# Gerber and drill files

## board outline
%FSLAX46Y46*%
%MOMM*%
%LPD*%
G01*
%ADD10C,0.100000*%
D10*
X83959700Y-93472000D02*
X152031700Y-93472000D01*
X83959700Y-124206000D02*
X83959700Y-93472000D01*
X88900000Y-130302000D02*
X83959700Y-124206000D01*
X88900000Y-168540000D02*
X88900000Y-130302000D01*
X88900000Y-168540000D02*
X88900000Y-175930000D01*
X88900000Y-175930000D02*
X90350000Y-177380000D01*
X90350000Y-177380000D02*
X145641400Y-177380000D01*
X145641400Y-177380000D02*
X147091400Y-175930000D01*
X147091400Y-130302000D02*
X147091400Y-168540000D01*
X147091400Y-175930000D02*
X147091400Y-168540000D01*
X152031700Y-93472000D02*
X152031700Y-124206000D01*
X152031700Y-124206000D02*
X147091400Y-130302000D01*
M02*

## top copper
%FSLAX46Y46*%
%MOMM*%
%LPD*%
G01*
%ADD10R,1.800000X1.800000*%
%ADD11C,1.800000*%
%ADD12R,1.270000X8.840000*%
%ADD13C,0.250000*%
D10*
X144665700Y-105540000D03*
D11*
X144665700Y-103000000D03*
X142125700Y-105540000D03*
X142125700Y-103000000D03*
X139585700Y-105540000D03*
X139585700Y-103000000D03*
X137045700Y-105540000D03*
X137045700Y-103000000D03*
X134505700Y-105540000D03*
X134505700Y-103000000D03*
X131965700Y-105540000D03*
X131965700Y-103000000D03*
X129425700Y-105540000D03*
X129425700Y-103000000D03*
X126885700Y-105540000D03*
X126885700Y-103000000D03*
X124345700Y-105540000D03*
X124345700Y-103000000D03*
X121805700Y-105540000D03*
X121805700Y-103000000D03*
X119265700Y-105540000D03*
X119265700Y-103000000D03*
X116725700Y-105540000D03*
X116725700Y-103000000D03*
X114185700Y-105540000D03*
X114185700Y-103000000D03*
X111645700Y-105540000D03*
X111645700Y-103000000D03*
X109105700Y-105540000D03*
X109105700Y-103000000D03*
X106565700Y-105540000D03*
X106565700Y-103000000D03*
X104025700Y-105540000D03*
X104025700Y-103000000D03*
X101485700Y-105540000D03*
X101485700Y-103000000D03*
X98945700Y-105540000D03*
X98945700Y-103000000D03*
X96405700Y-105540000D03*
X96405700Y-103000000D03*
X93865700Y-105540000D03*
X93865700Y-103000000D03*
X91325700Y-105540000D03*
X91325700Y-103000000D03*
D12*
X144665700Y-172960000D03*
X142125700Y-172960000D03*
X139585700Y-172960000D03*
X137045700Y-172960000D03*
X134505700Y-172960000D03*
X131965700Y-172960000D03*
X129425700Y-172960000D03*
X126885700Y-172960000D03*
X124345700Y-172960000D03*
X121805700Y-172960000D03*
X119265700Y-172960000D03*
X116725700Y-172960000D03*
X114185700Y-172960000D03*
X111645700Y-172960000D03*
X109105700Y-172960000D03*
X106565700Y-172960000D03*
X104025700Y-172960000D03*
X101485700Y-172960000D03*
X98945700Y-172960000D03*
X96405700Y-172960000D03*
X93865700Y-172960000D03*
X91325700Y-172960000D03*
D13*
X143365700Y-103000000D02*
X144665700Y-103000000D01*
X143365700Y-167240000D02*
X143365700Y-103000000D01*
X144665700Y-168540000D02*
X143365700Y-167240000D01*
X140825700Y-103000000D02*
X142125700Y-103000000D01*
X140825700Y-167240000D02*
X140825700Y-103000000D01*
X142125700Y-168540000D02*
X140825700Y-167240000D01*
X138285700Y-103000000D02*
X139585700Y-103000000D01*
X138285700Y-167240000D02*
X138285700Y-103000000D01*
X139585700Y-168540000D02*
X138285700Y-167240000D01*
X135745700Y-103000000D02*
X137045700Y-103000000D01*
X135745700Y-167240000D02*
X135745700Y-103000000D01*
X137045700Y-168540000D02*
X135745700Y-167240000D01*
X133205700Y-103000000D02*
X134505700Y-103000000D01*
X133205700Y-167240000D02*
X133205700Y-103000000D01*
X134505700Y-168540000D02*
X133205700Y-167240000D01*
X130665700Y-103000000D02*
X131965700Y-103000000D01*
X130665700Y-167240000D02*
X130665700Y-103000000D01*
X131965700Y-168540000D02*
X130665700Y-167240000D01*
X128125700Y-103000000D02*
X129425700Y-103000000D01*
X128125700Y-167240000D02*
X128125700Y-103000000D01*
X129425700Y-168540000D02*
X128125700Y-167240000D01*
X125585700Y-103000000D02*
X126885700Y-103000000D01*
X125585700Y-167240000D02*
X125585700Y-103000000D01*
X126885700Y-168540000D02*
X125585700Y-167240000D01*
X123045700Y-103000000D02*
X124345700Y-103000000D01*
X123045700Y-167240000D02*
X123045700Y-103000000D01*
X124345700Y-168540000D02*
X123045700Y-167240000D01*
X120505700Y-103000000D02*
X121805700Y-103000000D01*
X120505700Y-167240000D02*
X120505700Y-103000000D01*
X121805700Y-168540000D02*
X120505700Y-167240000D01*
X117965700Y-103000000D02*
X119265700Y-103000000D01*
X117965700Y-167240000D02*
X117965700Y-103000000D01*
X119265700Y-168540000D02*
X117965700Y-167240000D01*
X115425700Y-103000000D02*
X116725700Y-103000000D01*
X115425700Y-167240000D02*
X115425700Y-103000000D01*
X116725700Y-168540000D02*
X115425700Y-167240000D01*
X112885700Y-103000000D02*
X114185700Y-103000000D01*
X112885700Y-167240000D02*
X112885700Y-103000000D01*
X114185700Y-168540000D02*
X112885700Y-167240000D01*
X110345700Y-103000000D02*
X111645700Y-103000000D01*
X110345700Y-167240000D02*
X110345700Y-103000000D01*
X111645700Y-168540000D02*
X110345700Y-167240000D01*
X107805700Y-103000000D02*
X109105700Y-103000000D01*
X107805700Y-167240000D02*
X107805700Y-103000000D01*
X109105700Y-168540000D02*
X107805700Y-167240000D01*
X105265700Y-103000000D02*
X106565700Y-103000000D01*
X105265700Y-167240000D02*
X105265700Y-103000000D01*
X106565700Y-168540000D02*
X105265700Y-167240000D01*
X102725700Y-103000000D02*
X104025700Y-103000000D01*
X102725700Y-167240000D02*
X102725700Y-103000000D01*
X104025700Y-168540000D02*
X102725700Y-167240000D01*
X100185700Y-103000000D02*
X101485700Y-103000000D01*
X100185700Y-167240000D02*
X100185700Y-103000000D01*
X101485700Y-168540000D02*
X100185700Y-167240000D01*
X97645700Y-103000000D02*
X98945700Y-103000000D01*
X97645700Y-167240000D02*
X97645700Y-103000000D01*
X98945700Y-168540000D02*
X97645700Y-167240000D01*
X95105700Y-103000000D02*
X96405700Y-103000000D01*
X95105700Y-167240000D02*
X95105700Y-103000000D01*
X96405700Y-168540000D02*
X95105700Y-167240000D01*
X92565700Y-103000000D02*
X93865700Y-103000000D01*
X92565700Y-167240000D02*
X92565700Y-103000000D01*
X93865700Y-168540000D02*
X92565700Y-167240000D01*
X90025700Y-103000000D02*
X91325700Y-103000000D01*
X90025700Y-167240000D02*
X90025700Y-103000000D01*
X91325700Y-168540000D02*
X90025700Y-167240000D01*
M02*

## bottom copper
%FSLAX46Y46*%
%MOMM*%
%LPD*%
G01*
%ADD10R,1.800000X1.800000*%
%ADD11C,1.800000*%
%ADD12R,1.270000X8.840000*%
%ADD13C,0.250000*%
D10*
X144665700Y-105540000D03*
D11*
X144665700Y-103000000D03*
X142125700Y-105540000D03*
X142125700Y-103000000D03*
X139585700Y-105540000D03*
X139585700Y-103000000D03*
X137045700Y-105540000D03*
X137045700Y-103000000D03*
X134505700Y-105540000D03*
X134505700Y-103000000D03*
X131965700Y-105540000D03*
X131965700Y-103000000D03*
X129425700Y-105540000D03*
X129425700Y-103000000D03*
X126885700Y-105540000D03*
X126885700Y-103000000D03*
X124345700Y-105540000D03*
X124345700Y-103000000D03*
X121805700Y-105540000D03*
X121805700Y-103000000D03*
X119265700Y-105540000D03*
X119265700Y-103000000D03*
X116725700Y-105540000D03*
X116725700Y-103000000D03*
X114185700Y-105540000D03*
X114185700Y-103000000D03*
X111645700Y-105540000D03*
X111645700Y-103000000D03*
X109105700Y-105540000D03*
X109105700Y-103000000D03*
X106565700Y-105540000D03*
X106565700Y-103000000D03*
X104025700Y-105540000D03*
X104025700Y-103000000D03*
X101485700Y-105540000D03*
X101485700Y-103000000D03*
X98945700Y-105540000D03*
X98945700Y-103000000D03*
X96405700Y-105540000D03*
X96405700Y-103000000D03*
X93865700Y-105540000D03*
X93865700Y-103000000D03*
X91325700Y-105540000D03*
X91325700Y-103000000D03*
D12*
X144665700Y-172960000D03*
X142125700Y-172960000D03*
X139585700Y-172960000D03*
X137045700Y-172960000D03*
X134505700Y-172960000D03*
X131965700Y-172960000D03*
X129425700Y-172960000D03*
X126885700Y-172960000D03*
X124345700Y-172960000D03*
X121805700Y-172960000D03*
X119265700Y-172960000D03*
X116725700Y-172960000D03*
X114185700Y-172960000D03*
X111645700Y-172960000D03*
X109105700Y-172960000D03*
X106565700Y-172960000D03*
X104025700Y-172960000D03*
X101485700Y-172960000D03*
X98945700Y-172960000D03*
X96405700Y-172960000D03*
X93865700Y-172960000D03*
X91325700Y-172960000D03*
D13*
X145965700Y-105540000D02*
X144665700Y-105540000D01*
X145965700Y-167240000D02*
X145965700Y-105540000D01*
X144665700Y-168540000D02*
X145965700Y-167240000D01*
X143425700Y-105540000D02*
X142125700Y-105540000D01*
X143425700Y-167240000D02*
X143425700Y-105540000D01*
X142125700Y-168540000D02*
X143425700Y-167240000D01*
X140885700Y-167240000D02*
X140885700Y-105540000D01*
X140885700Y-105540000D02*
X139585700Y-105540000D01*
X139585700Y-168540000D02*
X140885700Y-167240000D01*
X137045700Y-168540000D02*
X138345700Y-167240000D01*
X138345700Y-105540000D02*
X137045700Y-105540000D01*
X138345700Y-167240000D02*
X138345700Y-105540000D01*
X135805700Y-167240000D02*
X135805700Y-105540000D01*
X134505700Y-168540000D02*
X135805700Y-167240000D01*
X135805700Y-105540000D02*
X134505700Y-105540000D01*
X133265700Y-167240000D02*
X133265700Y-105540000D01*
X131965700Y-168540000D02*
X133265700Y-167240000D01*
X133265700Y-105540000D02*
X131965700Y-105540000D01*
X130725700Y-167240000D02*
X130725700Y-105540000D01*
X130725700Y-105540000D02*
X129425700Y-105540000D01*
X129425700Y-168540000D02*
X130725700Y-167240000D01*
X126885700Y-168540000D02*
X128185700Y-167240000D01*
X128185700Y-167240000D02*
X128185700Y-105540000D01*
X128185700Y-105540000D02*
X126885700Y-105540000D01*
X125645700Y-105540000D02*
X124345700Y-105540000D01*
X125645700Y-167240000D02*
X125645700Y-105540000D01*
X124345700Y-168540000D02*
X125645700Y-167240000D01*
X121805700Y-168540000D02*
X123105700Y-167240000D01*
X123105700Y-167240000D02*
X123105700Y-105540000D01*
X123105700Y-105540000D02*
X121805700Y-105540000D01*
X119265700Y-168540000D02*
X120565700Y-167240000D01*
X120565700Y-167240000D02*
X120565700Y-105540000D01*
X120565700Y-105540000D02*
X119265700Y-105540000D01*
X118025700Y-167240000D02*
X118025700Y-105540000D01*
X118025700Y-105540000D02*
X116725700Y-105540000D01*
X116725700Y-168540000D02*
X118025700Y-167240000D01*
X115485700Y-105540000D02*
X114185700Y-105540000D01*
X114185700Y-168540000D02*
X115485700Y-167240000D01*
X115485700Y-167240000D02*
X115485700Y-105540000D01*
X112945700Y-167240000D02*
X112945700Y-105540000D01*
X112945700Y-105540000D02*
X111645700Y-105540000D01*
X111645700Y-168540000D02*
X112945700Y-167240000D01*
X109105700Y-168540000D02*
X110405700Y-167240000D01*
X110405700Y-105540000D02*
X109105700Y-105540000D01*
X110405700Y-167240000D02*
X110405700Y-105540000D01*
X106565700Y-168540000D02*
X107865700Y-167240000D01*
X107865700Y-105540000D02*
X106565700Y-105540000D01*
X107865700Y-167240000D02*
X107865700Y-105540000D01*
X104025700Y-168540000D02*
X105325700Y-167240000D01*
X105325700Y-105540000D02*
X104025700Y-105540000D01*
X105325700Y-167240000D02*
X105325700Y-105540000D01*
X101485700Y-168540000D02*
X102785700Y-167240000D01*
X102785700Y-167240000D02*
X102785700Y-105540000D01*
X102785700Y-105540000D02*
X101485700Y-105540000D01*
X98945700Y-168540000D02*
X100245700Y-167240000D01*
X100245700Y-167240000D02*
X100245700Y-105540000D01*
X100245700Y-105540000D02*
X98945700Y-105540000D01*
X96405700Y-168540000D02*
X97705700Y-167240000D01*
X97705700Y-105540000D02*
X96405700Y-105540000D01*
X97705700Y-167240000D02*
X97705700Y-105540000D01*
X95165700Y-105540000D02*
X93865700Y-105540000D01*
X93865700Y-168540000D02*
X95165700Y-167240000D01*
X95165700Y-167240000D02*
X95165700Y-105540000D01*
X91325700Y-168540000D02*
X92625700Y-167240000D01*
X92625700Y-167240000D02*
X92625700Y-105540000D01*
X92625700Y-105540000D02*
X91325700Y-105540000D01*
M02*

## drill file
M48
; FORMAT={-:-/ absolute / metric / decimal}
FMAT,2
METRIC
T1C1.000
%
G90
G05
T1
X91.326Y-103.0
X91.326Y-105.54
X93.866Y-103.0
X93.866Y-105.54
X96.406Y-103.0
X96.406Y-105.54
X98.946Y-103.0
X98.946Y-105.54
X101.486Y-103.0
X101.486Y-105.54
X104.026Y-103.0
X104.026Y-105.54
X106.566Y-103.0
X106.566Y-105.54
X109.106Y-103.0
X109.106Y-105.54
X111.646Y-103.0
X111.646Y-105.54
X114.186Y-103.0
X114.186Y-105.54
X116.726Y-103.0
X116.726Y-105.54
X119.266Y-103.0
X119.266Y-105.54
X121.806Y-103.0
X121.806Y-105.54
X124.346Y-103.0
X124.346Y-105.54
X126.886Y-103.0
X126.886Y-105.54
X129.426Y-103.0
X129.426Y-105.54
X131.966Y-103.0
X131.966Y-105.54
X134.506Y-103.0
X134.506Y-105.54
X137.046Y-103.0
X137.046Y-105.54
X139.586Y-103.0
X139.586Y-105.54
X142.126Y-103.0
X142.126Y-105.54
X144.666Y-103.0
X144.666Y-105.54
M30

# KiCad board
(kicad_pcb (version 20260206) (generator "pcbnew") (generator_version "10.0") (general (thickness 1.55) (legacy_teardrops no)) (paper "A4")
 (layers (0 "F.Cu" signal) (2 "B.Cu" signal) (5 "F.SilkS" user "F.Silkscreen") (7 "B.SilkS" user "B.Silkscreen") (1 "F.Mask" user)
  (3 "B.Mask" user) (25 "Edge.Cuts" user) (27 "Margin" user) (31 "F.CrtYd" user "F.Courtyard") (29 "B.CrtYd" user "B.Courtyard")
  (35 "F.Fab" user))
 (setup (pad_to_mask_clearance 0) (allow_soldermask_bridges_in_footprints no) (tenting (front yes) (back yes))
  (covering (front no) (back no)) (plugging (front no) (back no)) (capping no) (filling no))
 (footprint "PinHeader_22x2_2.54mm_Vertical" (layer "F.Cu") (at 0 0)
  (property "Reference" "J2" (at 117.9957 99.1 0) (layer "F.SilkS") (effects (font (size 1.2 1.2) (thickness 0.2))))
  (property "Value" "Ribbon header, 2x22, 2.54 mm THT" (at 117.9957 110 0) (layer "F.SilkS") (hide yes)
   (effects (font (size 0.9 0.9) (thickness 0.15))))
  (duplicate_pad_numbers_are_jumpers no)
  (pad "1" thru_hole rect (at 144.6657 105.54) (size 1.8 1.8) (drill 1) (layers "*.Cu" "*.Mask") (remove_unused_layers no) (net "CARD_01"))
  (pad "2" thru_hole circle (at 144.6657 103) (size 1.8 1.8) (drill 1) (layers "*.Cu" "*.Mask") (remove_unused_layers no) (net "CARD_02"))
  (pad "3" thru_hole circle (at 142.1257 105.54) (size 1.8 1.8) (drill 1) (layers "*.Cu" "*.Mask") (remove_unused_layers no) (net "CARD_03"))
  (pad "4" thru_hole circle (at 142.1257 103) (size 1.8 1.8) (drill 1) (layers "*.Cu" "*.Mask") (remove_unused_layers no) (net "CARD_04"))
  (pad "5" thru_hole circle (at 139.5857 105.54) (size 1.8 1.8) (drill 1) (layers "*.Cu" "*.Mask") (remove_unused_layers no) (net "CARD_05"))
  (pad "6" thru_hole circle (at 139.5857 103) (size 1.8 1.8) (drill 1) (layers "*.Cu" "*.Mask") (remove_unused_layers no) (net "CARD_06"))
  (pad "7" thru_hole circle (at 137.0457 105.54) (size 1.8 1.8) (drill 1) (layers "*.Cu" "*.Mask") (remove_unused_layers no) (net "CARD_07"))
  (pad "8" thru_hole circle (at 137.0457 103) (size 1.8 1.8) (drill 1) (layers "*.Cu" "*.Mask") (remove_unused_layers no) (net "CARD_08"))
  (pad "9" thru_hole circle (at 134.5057 105.54) (size 1.8 1.8) (drill 1) (layers "*.Cu" "*.Mask") (remove_unused_layers no) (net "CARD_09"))
  (pad "10" thru_hole circle (at 134.5057 103) (size 1.8 1.8) (drill 1) (layers "*.Cu" "*.Mask") (remove_unused_layers no) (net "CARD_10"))
  (pad "11" thru_hole circle (at 131.9657 105.54) (size 1.8 1.8) (drill 1) (layers "*.Cu" "*.Mask") (remove_unused_layers no)
   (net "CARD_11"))
  (pad "12" thru_hole circle (at 131.9657 103) (size 1.8 1.8) (drill 1) (layers "*.Cu" "*.Mask") (remove_unused_layers no) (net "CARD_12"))
  (pad "13" thru_hole circle (at 129.4257 105.54) (size 1.8 1.8) (drill 1) (layers "*.Cu" "*.Mask") (remove_unused_layers no)
   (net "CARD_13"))
  (pad "14" thru_hole circle (at 129.4257 103) (size 1.8 1.8) (drill 1) (layers "*.Cu" "*.Mask") (remove_unused_layers no) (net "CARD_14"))
  (pad "15" thru_hole circle (at 126.8857 105.54) (size 1.8 1.8) (drill 1) (layers "*.Cu" "*.Mask") (remove_unused_layers no)
   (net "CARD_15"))
  (pad "16" thru_hole circle (at 126.8857 103) (size 1.8 1.8) (drill 1) (layers "*.Cu" "*.Mask") (remove_unused_layers no) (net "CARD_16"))
  (pad "17" thru_hole circle (at 124.3457 105.54) (size 1.8 1.8) (drill 1) (layers "*.Cu" "*.Mask") (remove_unused_layers no)
   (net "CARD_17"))
  (pad "18" thru_hole circle (at 124.3457 103) (size 1.8 1.8) (drill 1) (layers "*.Cu" "*.Mask") (remove_unused_layers no) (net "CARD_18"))
  (pad "19" thru_hole circle (at 121.8057 105.54) (size 1.8 1.8) (drill 1) (layers "*.Cu" "*.Mask") (remove_unused_layers no)
   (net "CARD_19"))
  (pad "20" thru_hole circle (at 121.8057 103) (size 1.8 1.8) (drill 1) (layers "*.Cu" "*.Mask") (remove_unused_layers no) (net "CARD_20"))
  (pad "21" thru_hole circle (at 119.2657 105.54) (size 1.8 1.8) (drill 1) (layers "*.Cu" "*.Mask") (remove_unused_layers no)
   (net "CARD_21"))
  (pad "22" thru_hole circle (at 119.2657 103) (size 1.8 1.8) (drill 1) (layers "*.Cu" "*.Mask") (remove_unused_layers no) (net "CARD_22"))
  (pad "23" thru_hole circle (at 116.7257 105.54) (size 1.8 1.8) (drill 1) (layers "*.Cu" "*.Mask") (remove_unused_layers no)
   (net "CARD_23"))
  (pad "24" thru_hole circle (at 116.7257 103) (size 1.8 1.8) (drill 1) (layers "*.Cu" "*.Mask") (remove_unused_layers no) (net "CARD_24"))
  (pad "25" thru_hole circle (at 114.1857 105.54) (size 1.8 1.8) (drill 1) (layers "*.Cu" "*.Mask") (remove_unused_layers no)
   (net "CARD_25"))
  (pad "26" thru_hole circle (at 114.1857 103) (size 1.8 1.8) (drill 1) (layers "*.Cu" "*.Mask") (remove_unused_layers no) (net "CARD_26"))
  (pad "27" thru_hole circle (at 111.6457 105.54) (size 1.8 1.8) (drill 1) (layers "*.Cu" "*.Mask") (remove_unused_layers no)
   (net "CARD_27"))
  (pad "28" thru_hole circle (at 111.6457 103) (size 1.8 1.8) (drill 1) (layers "*.Cu" "*.Mask") (remove_unused_layers no) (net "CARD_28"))
  (pad "29" thru_hole circle (at 109.1057 105.54) (size 1.8 1.8) (drill 1) (layers "*.Cu" "*.Mask") (remove_unused_layers no)
   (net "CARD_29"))
  (pad "30" thru_hole circle (at 109.1057 103) (size 1.8 1.8) (drill 1) (layers "*.Cu" "*.Mask") (remove_unused_layers no) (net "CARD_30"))
  (pad "31" thru_hole circle (at 106.5657 105.54) (size 1.8 1.8) (drill 1) (layers "*.Cu" "*.Mask") (remove_unused_layers no)
   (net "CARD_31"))
  (pad "32" thru_hole circle (at 106.5657 103) (size 1.8 1.8) (drill 1) (layers "*.Cu" "*.Mask") (remove_unused_layers no) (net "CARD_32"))
  (pad "33" thru_hole circle (at 104.0257 105.54) (size 1.8 1.8) (drill 1) (layers "*.Cu" "*.Mask") (remove_unused_layers no)
   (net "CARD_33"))
  (pad "34" thru_hole circle (at 104.0257 103) (size 1.8 1.8) (drill 1) (layers "*.Cu" "*.Mask") (remove_unused_layers no) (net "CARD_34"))
  (pad "35" thru_hole circle (at 101.4857 105.54) (size 1.8 1.8) (drill 1) (layers "*.Cu" "*.Mask") (remove_unused_layers no)
   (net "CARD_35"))
  (pad "36" thru_hole circle (at 101.4857 103) (size 1.8 1.8) (drill 1) (layers "*.Cu" "*.Mask") (remove_unused_layers no) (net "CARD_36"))
  (pad "37" thru_hole circle (at 98.9457 105.54) (size 1.8 1.8) (drill 1) (layers "*.Cu" "*.Mask") (remove_unused_layers no) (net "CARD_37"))
  (pad "38" thru_hole circle (at 98.9457 103) (size 1.8 1.8) (drill 1) (layers "*.Cu" "*.Mask") (remove_unused_layers no) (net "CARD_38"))
  (pad "39" thru_hole circle (at 96.4057 105.54) (size 1.8 1.8) (drill 1) (layers "*.Cu" "*.Mask") (remove_unused_layers no) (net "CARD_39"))
  (pad "40" thru_hole circle (at 96.4057 103) (size 1.8 1.8) (drill 1) (layers "*.Cu" "*.Mask") (remove_unused_layers no) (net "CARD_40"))
  (pad "41" thru_hole circle (at 93.8657 105.54) (size 1.8 1.8) (drill 1) (layers "*.Cu" "*.Mask") (remove_unused_layers no) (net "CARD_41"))
  (pad "42" thru_hole circle (at 93.8657 103) (size 1.8 1.8) (drill 1) (layers "*.Cu" "*.Mask") (remove_unused_layers no) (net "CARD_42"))
  (pad "43" thru_hole circle (at 91.3257 105.54) (size 1.8 1.8) (drill 1) (layers "*.Cu" "*.Mask") (remove_unused_layers no) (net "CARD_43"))
  (pad "44" thru_hole circle (at 91.3257 103) (size 1.8 1.8) (drill 1) (layers "*.Cu" "*.Mask") (remove_unused_layers no) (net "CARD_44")))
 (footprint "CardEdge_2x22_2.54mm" (layer "F.Cu") (at 0 -15)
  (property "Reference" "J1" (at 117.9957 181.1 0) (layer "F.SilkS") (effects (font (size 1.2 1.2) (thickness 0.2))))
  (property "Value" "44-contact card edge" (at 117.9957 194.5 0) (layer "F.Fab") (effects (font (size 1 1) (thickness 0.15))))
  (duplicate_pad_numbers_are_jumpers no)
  (pad "1" connect rect (at 144.6657 187.96) (size 1.27 8.84) (layers "B.Cu" "B.Mask") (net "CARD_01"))
  (pad "2" connect rect (at 144.6657 187.96) (size 1.27 8.84) (layers "F.Cu" "F.Mask") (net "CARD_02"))
  (pad "3" connect rect (at 142.1257 187.96) (size 1.27 8.84) (layers "B.Cu" "B.Mask") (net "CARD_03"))
  (pad "4" connect rect (at 142.1257 187.96) (size 1.27 8.84) (layers "F.Cu" "F.Mask") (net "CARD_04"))
  (pad "5" connect rect (at 139.5857 187.96) (size 1.27 8.84) (layers "B.Cu" "B.Mask") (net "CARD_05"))
  (pad "6" connect rect (at 139.5857 187.96) (size 1.27 8.84) (layers "F.Cu" "F.Mask") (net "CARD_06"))
  (pad "7" connect rect (at 137.0457 187.96) (size 1.27 8.84) (layers "B.Cu" "B.Mask") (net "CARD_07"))
  (pad "8" connect rect (at 137.0457 187.96) (size 1.27 8.84) (layers "F.Cu" "F.Mask") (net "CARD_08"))
  (pad "9" connect rect (at 134.5057 187.96) (size 1.27 8.84) (layers "B.Cu" "B.Mask") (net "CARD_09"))
  (pad "10" connect rect (at 134.5057 187.96) (size 1.27 8.84) (layers "F.Cu" "F.Mask") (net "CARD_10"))
  (pad "11" connect rect (at 131.9657 187.96) (size 1.27 8.84) (layers "B.Cu" "B.Mask") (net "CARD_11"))
  (pad "12" connect rect (at 131.9657 187.96) (size 1.27 8.84) (layers "F.Cu" "F.Mask") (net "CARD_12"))
  (pad "13" connect rect (at 129.4257 187.96) (size 1.27 8.84) (layers "B.Cu" "B.Mask") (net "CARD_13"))
  (pad "14" connect rect (at 129.4257 187.96) (size 1.27 8.84) (layers "F.Cu" "F.Mask") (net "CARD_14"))
  (pad "15" connect rect (at 126.8857 187.96) (size 1.27 8.84) (layers "B.Cu" "B.Mask") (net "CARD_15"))
  (pad "16" connect rect (at 126.8857 187.96) (size 1.27 8.84) (layers "F.Cu" "F.Mask") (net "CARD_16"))
  (pad "17" connect rect (at 124.3457 187.96) (size 1.27 8.84) (layers "B.Cu" "B.Mask") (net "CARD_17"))
  (pad "18" connect rect (at 124.3457 187.96) (size 1.27 8.84) (layers "F.Cu" "F.Mask") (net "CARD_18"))
  (pad "19" connect rect (at 121.8057 187.96) (size 1.27 8.84) (layers "B.Cu" "B.Mask") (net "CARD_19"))
  (pad "20" connect rect (at 121.8057 187.96) (size 1.27 8.84) (layers "F.Cu" "F.Mask") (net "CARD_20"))
  (pad "21" connect rect (at 119.2657 187.96) (size 1.27 8.84) (layers "B.Cu" "B.Mask") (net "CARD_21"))
  (pad "22" connect rect (at 119.2657 187.96) (size 1.27 8.84) (layers "F.Cu" "F.Mask") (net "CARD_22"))
  (pad "23" connect rect (at 116.7257 187.96) (size 1.27 8.84) (layers "B.Cu" "B.Mask") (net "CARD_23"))
  (pad "24" connect rect (at 116.7257 187.96) (size 1.27 8.84) (layers "F.Cu" "F.Mask") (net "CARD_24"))
  (pad "25" connect rect (at 114.1857 187.96) (size 1.27 8.84) (layers "B.Cu" "B.Mask") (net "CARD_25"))
  (pad "26" connect rect (at 114.1857 187.96) (size 1.27 8.84) (layers "F.Cu" "F.Mask") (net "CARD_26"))
  (pad "27" connect rect (at 111.6457 187.96) (size 1.27 8.84) (layers "B.Cu" "B.Mask") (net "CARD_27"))
  (pad "28" connect rect (at 111.6457 187.96) (size 1.27 8.84) (layers "F.Cu" "F.Mask") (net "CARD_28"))
  (pad "29" connect rect (at 109.1057 187.96) (size 1.27 8.84) (layers "B.Cu" "B.Mask") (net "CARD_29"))
  (pad "30" connect rect (at 109.1057 187.96) (size 1.27 8.84) (layers "F.Cu" "F.Mask") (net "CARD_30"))
  (pad "31" connect rect (at 106.5657 187.96) (size 1.27 8.84) (layers "B.Cu" "B.Mask") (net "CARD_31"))
  (pad "32" connect rect (at 106.5657 187.96) (size 1.27 8.84) (layers "F.Cu" "F.Mask") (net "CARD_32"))
  (pad "33" connect rect (at 104.0257 187.96) (size 1.27 8.84) (layers "B.Cu" "B.Mask") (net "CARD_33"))
  (pad "34" connect rect (at 104.0257 187.96) (size 1.27 8.84) (layers "F.Cu" "F.Mask") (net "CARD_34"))
  (pad "35" connect rect (at 101.4857 187.96) (size 1.27 8.84) (layers "B.Cu" "B.Mask") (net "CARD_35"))
  (pad "36" connect rect (at 101.4857 187.96) (size 1.27 8.84) (layers "F.Cu" "F.Mask") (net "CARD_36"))
  (pad "37" connect rect (at 98.9457 187.96) (size 1.27 8.84) (layers "B.Cu" "B.Mask") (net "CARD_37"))
  (pad "38" connect rect (at 98.9457 187.96) (size 1.27 8.84) (layers "F.Cu" "F.Mask") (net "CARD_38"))
  (pad "39" connect rect (at 96.4057 187.96) (size 1.27 8.84) (layers "B.Cu" "B.Mask") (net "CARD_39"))
  (pad "40" connect rect (at 96.4057 187.96) (size 1.27 8.84) (layers "F.Cu" "F.Mask") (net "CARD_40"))
  (pad "41" connect rect (at 93.8657 187.96) (size 1.27 8.84) (layers "B.Cu" "B.Mask") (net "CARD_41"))
  (pad "42" connect rect (at 93.8657 187.96) (size 1.27 8.84) (layers "F.Cu" "F.Mask") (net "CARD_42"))
  (pad "43" connect rect (at 91.3257 187.96) (size 1.27 8.84) (layers "B.Cu" "B.Mask") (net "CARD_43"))
  (pad "44" connect rect (at 91.3257 187.96) (size 1.27 8.84) (layers "F.Cu" "F.Mask") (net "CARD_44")))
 (gr_line (start 83.9597 93.472) (end 152.0317 93.472) (stroke (width 0.1) (type solid)) (layer "Edge.Cuts"))
 (gr_line (start 83.9597 124.206) (end 83.9597 93.472) (stroke (width 0.1) (type solid)) (layer "Edge.Cuts"))
 (gr_line (start 88.9 130.302) (end 83.9597 124.206) (stroke (width 0.1) (type solid)) (layer "Edge.Cuts"))
 (gr_line (start 88.9 168.54) (end 88.9 130.302) (stroke (width 0.1) (type solid)) (layer "Edge.Cuts"))
 (gr_line (start 88.9 168.54) (end 88.9 175.93) (stroke (width 0.1) (type solid)) (layer "Edge.Cuts"))
 (gr_line (start 88.9 175.93) (end 90.35 177.38) (stroke (width 0.1) (type solid)) (layer "Edge.Cuts"))
 (gr_line (start 90.35 177.38) (end 145.6414 177.38) (stroke (width 0.1) (type solid)) (layer "Edge.Cuts"))
 (gr_line (start 145.6414 177.38) (end 147.0914 175.93) (stroke (width 0.1) (type solid)) (layer "Edge.Cuts"))
 (gr_line (start 147.0914 130.302) (end 147.0914 168.54) (stroke (width 0.1) (type solid)) (layer "Edge.Cuts"))
 (gr_line (start 147.0914 175.93) (end 147.0914 168.54) (stroke (width 0.1) (type solid)) (layer "Edge.Cuts"))
 (gr_line (start 152.0317 93.472) (end 152.0317 124.206) (stroke (width 0.1) (type solid)) (layer "Edge.Cuts"))
 (gr_line (start 152.0317 124.206) (end 147.0914 130.302) (stroke (width 0.1) (type solid)) (layer "Edge.Cuts"))
 (segment (start 145.9657 105.54) (end 144.6657 105.54) (width 0.25) (layer "B.Cu") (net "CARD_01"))
 (segment (start 145.9657 167.24) (end 145.9657 105.54) (width 0.25) (layer "B.Cu") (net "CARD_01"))
 (segment (start 144.6657 168.54) (end 145.9657 167.24) (width 0.25) (layer "B.Cu") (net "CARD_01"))
 (segment (start 143.3657 103) (end 144.6657 103) (width 0.25) (layer "F.Cu") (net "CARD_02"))
 (segment (start 143.3657 167.24) (end 143.3657 103) (width 0.25) (layer "F.Cu") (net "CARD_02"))
 (segment (start 144.6657 168.54) (end 143.3657 167.24) (width 0.25) (layer "F.Cu") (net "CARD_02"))
 (segment (start 143.4257 105.54) (end 142.1257 105.54) (width 0.25) (layer "B.Cu") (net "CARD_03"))
 (segment (start 143.4257 167.24) (end 143.4257 105.54) (width 0.25) (layer "B.Cu") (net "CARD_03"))
 (segment (start 142.1257 168.54) (end 143.4257 167.24) (width 0.25) (layer "B.Cu") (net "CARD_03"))
 (segment (start 140.8257 103) (end 142.1257 103) (width 0.25) (layer "F.Cu") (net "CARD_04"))
 (segment (start 140.8257 167.24) (end 140.8257 103) (width 0.25) (layer "F.Cu") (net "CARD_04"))
 (segment (start 142.1257 168.54) (end 140.8257 167.24) (width 0.25) (layer "F.Cu") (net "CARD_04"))
 (segment (start 140.8857 167.24) (end 140.8857 105.54) (width 0.25) (layer "B.Cu") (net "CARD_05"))
 (segment (start 140.8857 105.54) (end 139.5857 105.54) (width 0.25) (layer "B.Cu") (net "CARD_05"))
 (segment (start 139.5857 168.54) (end 140.8857 167.24) (width 0.25) (layer "B.Cu") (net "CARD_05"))
 (segment (start 138.2857 103) (end 139.5857 103) (width 0.25) (layer "F.Cu") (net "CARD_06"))
 (segment (start 138.2857 167.24) (end 138.2857 103) (width 0.25) (layer "F.Cu") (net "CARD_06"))
 (segment (start 139.5857 168.54) (end 138.2857 167.24) (width 0.25) (layer "F.Cu") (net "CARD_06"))
 (segment (start 137.0457 168.54) (end 138.3457 167.24) (width 0.25) (layer "B.Cu") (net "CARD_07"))
 (segment (start 138.3457 105.54) (end 137.0457 105.54) (width 0.25) (layer "B.Cu") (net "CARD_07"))
 (segment (start 138.3457 167.24) (end 138.3457 105.54) (width 0.25) (layer "B.Cu") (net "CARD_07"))
 (segment (start 135.7457 103) (end 137.0457 103) (width 0.25) (layer "F.Cu") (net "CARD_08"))
 (segment (start 135.7457 167.24) (end 135.7457 103) (width 0.25) (layer "F.Cu") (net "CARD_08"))
 (segment (start 137.0457 168.54) (end 135.7457 167.24) (width 0.25) (layer "F.Cu") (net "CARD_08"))
 (segment (start 135.8057 167.24) (end 135.8057 105.54) (width 0.25) (layer "B.Cu") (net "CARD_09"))
 (segment (start 134.5057 168.54) (end 135.8057 167.24) (width 0.25) (layer "B.Cu") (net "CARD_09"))
 (segment (start 135.8057 105.54) (end 134.5057 105.54) (width 0.25) (layer "B.Cu") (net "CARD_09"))
 (segment (start 133.2057 103) (end 134.5057 103) (width 0.25) (layer "F.Cu") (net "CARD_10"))
 (segment (start 133.2057 167.24) (end 133.2057 103) (width 0.25) (layer "F.Cu") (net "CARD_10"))
 (segment (start 134.5057 168.54) (end 133.2057 167.24) (width 0.25) (layer "F.Cu") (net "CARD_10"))
 (segment (start 133.2657 167.24) (end 133.2657 105.54) (width 0.25) (layer "B.Cu") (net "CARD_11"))
 (segment (start 131.9657 168.54) (end 133.2657 167.24) (width 0.25) (layer "B.Cu") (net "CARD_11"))
 (segment (start 133.2657 105.54) (end 131.9657 105.54) (width 0.25) (layer "B.Cu") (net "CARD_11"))
 (segment (start 130.6657 103) (end 131.9657 103) (width 0.25) (layer "F.Cu") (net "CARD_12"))
 (segment (start 130.6657 167.24) (end 130.6657 103) (width 0.25) (layer "F.Cu") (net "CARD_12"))
 (segment (start 131.9657 168.54) (end 130.6657 167.24) (width 0.25) (layer "F.Cu") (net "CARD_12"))
 (segment (start 130.7257 167.24) (end 130.7257 105.54) (width 0.25) (layer "B.Cu") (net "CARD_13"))
 (segment (start 130.7257 105.54) (end 129.4257 105.54) (width 0.25) (layer "B.Cu") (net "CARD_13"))
 (segment (start 129.4257 168.54) (end 130.7257 167.24) (width 0.25) (layer "B.Cu") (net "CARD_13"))
 (segment (start 128.1257 103) (end 129.4257 103) (width 0.25) (layer "F.Cu") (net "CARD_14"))
 (segment (start 128.1257 167.24) (end 128.1257 103) (width 0.25) (layer "F.Cu") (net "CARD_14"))
 (segment (start 129.4257 168.54) (end 128.1257 167.24) (width 0.25) (layer "F.Cu") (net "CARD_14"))
 (segment (start 126.8857 168.54) (end 128.1857 167.24) (width 0.25) (layer "B.Cu") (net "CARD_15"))
 (segment (start 128.1857 167.24) (end 128.1857 105.54) (width 0.25) (layer "B.Cu") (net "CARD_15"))
 (segment (start 128.1857 105.54) (end 126.8857 105.54) (width 0.25) (layer "B.Cu") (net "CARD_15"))
 (segment (start 125.5857 103) (end 126.8857 103) (width 0.25) (layer "F.Cu") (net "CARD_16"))
 (segment (start 125.5857 167.24) (end 125.5857 103) (width 0.25) (layer "F.Cu") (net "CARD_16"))
 (segment (start 126.8857 168.54) (end 125.5857 167.24) (width 0.25) (layer "F.Cu") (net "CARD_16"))
 (segment (start 125.6457 105.54) (end 124.3457 105.54) (width 0.25) (layer "B.Cu") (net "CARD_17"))
 (segment (start 125.6457 167.24) (end 125.6457 105.54) (width 0.25) (layer "B.Cu") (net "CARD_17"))
 (segment (start 124.3457 168.54) (end 125.6457 167.24) (width 0.25) (layer "B.Cu") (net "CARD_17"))
 (segment (start 123.0457 103) (end 124.3457 103) (width 0.25) (layer "F.Cu") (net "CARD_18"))
 (segment (start 123.0457 167.24) (end 123.0457 103) (width 0.25) (layer "F.Cu") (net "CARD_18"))
 (segment (start 124.3457 168.54) (end 123.0457 167.24) (width 0.25) (layer "F.Cu") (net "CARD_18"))
 (segment (start 121.8057 168.54) (end 123.1057 167.24) (width 0.25) (layer "B.Cu") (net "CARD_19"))
 (segment (start 123.1057 167.24) (end 123.1057 105.54) (width 0.25) (layer "B.Cu") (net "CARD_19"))
 (segment (start 123.1057 105.54) (end 121.8057 105.54) (width 0.25) (layer "B.Cu") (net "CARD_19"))
 (segment (start 120.5057 103) (end 121.8057 103) (width 0.25) (layer "F.Cu") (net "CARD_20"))
 (segment (start 120.5057 167.24) (end 120.5057 103) (width 0.25) (layer "F.Cu") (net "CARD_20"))
 (segment (start 121.8057 168.54) (end 120.5057 167.24) (width 0.25) (layer "F.Cu") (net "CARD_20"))
 (segment (start 119.2657 168.54) (end 120.5657 167.24) (width 0.25) (layer "B.Cu") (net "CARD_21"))
 (segment (start 120.5657 167.24) (end 120.5657 105.54) (width 0.25) (layer "B.Cu") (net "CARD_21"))
 (segment (start 120.5657 105.54) (end 119.2657 105.54) (width 0.25) (layer "B.Cu") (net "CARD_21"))
 (segment (start 117.9657 103) (end 119.2657 103) (width 0.25) (layer "F.Cu") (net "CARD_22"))
 (segment (start 117.9657 167.24) (end 117.9657 103) (width 0.25) (layer "F.Cu") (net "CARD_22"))
 (segment (start 119.2657 168.54) (end 117.9657 167.24) (width 0.25) (layer "F.Cu") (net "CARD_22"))
 (segment (start 118.0257 167.24) (end 118.0257 105.54) (width 0.25) (layer "B.Cu") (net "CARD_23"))
 (segment (start 118.0257 105.54) (end 116.7257 105.54) (width 0.25) (layer "B.Cu") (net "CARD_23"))
 (segment (start 116.7257 168.54) (end 118.0257 167.24) (width 0.25) (layer "B.Cu") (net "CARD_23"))
 (segment (start 115.4257 103) (end 116.7257 103) (width 0.25) (layer "F.Cu") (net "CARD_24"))
 (segment (start 115.4257 167.24) (end 115.4257 103) (width 0.25) (layer "F.Cu") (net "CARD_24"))
 (segment (start 116.7257 168.54) (end 115.4257 167.24) (width 0.25) (layer "F.Cu") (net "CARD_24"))
 (segment (start 115.4857 105.54) (end 114.1857 105.54) (width 0.25) (layer "B.Cu") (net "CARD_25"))
 (segment (start 114.1857 168.54) (end 115.4857 167.24) (width 0.25) (layer "B.Cu") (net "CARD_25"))
 (segment (start 115.4857 167.24) (end 115.4857 105.54) (width 0.25) (layer "B.Cu") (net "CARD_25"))
 (segment (start 112.8857 103) (end 114.1857 103) (width 0.25) (layer "F.Cu") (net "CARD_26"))
 (segment (start 112.8857 167.24) (end 112.8857 103) (width 0.25) (layer "F.Cu") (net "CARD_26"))
 (segment (start 114.1857 168.54) (end 112.8857 167.24) (width 0.25) (layer "F.Cu") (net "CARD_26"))
 (segment (start 112.9457 167.24) (end 112.9457 105.54) (width 0.25) (layer "B.Cu") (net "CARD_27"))
 (segment (start 112.9457 105.54) (end 111.6457 105.54) (width 0.25) (layer "B.Cu") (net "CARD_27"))
 (segment (start 111.6457 168.54) (end 112.9457 167.24) (width 0.25) (layer "B.Cu") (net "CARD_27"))
 (segment (start 110.3457 103) (end 111.6457 103) (width 0.25) (layer "F.Cu") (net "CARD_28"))
 (segment (start 110.3457 167.24) (end 110.3457 103) (width 0.25) (layer "F.Cu") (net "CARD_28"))
 (segment (start 111.6457 168.54) (end 110.3457 167.24) (width 0.25) (layer "F.Cu") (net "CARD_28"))
 (segment (start 109.1057 168.54) (end 110.4057 167.24) (width 0.25) (layer "B.Cu") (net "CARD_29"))
 (segment (start 110.4057 105.54) (end 109.1057 105.54) (width 0.25) (layer "B.Cu") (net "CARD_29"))
 (segment (start 110.4057 167.24) (end 110.4057 105.54) (width 0.25) (layer "B.Cu") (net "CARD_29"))
 (segment (start 107.8057 103) (end 109.1057 103) (width 0.25) (layer "F.Cu") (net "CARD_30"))
 (segment (start 107.8057 167.24) (end 107.8057 103) (width 0.25) (layer "F.Cu") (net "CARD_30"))
 (segment (start 109.1057 168.54) (end 107.8057 167.24) (width 0.25) (layer "F.Cu") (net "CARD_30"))
 (segment (start 106.5657 168.54) (end 107.8657 167.24) (width 0.25) (layer "B.Cu") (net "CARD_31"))
 (segment (start 107.8657 105.54) (end 106.5657 105.54) (width 0.25) (layer "B.Cu") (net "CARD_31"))
 (segment (start 107.8657 167.24) (end 107.8657 105.54) (width 0.25) (layer "B.Cu") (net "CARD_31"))
 (segment (start 105.2657 103) (end 106.5657 103) (width 0.25) (layer "F.Cu") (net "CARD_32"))
 (segment (start 105.2657 167.24) (end 105.2657 103) (width 0.25) (layer "F.Cu") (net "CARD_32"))
 (segment (start 106.5657 168.54) (end 105.2657 167.24) (width 0.25) (layer "F.Cu") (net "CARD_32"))
 (segment (start 104.0257 168.54) (end 105.3257 167.24) (width 0.25) (layer "B.Cu") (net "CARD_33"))
 (segment (start 105.3257 105.54) (end 104.0257 105.54) (width 0.25) (layer "B.Cu") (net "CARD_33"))
 (segment (start 105.3257 167.24) (end 105.3257 105.54) (width 0.25) (layer "B.Cu") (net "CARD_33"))
 (segment (start 102.7257 103) (end 104.0257 103) (width 0.25) (layer "F.Cu") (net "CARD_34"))
 (segment (start 102.7257 167.24) (end 102.7257 103) (width 0.25) (layer "F.Cu") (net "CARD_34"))
 (segment (start 104.0257 168.54) (end 102.7257 167.24) (width 0.25) (layer "F.Cu") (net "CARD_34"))
 (segment (start 101.4857 168.54) (end 102.7857 167.24) (width 0.25) (layer "B.Cu") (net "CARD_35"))
 (segment (start 102.7857 167.24) (end 102.7857 105.54) (width 0.25) (layer "B.Cu") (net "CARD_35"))
 (segment (start 102.7857 105.54) (end 101.4857 105.54) (width 0.25) (layer "B.Cu") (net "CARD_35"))
 (segment (start 100.1857 103) (end 101.4857 103) (width 0.25) (layer "F.Cu") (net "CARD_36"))
 (segment (start 100.1857 167.24) (end 100.1857 103) (width 0.25) (layer "F.Cu") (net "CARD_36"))
 (segment (start 101.4857 168.54) (end 100.1857 167.24) (width 0.25) (layer "F.Cu") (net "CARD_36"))
 (segment (start 98.9457 168.54) (end 100.2457 167.24) (width 0.25) (layer "B.Cu") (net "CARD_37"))
 (segment (start 100.2457 167.24) (end 100.2457 105.54) (width 0.25) (layer "B.Cu") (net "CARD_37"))
 (segment (start 100.2457 105.54) (end 98.9457 105.54) (width 0.25) (layer "B.Cu") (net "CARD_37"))
 (segment (start 97.6457 103) (end 98.9457 103) (width 0.25) (layer "F.Cu") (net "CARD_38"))
 (segment (start 97.6457 167.24) (end 97.6457 103) (width 0.25) (layer "F.Cu") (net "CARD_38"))
 (segment (start 98.9457 168.54) (end 97.6457 167.24) (width 0.25) (layer "F.Cu") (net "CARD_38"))
 (segment (start 96.4057 168.54) (end 97.7057 167.24) (width 0.25) (layer "B.Cu") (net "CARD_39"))
 (segment (start 97.7057 105.54) (end 96.4057 105.54) (width 0.25) (layer "B.Cu") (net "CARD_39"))
 (segment (start 97.7057 167.24) (end 97.7057 105.54) (width 0.25) (layer "B.Cu") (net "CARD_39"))
 (segment (start 95.1057 103) (end 96.4057 103) (width 0.25) (layer "F.Cu") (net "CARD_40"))
 (segment (start 95.1057 167.24) (end 95.1057 103) (width 0.25) (layer "F.Cu") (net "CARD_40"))
 (segment (start 96.4057 168.54) (end 95.1057 167.24) (width 0.25) (layer "F.Cu") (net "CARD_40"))
 (segment (start 95.1657 105.54) (end 93.8657 105.54) (width 0.25) (layer "B.Cu") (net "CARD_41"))
 (segment (start 93.8657 168.54) (end 95.1657 167.24) (width 0.25) (layer "B.Cu") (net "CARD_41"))
 (segment (start 95.1657 167.24) (end 95.1657 105.54) (width 0.25) (layer "B.Cu") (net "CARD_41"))
 (segment (start 92.5657 103) (end 93.8657 103) (width 0.25) (layer "F.Cu") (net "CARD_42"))
 (segment (start 92.5657 167.24) (end 92.5657 103) (width 0.25) (layer "F.Cu") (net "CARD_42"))
 (segment (start 93.8657 168.54) (end 92.5657 167.24) (width 0.25) (layer "F.Cu") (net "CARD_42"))
 (segment (start 91.3257 168.54) (end 92.6257 167.24) (width 0.25) (layer "B.Cu") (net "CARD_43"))
 (segment (start 92.6257 167.24) (end 92.6257 105.54) (width 0.25) (layer "B.Cu") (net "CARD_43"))
 (segment (start 92.6257 105.54) (end 91.3257 105.54) (width 0.25) (layer "B.Cu") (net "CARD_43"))
 (segment (start 90.0257 103) (end 91.3257 103) (width 0.25) (layer "F.Cu") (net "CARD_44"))
 (segment (start 90.0257 167.24) (end 90.0257 103) (width 0.25) (layer "F.Cu") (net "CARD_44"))
 (segment (start 91.3257 168.54) (end 90.0257 167.24) (width 0.25) (layer "F.Cu") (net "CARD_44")))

